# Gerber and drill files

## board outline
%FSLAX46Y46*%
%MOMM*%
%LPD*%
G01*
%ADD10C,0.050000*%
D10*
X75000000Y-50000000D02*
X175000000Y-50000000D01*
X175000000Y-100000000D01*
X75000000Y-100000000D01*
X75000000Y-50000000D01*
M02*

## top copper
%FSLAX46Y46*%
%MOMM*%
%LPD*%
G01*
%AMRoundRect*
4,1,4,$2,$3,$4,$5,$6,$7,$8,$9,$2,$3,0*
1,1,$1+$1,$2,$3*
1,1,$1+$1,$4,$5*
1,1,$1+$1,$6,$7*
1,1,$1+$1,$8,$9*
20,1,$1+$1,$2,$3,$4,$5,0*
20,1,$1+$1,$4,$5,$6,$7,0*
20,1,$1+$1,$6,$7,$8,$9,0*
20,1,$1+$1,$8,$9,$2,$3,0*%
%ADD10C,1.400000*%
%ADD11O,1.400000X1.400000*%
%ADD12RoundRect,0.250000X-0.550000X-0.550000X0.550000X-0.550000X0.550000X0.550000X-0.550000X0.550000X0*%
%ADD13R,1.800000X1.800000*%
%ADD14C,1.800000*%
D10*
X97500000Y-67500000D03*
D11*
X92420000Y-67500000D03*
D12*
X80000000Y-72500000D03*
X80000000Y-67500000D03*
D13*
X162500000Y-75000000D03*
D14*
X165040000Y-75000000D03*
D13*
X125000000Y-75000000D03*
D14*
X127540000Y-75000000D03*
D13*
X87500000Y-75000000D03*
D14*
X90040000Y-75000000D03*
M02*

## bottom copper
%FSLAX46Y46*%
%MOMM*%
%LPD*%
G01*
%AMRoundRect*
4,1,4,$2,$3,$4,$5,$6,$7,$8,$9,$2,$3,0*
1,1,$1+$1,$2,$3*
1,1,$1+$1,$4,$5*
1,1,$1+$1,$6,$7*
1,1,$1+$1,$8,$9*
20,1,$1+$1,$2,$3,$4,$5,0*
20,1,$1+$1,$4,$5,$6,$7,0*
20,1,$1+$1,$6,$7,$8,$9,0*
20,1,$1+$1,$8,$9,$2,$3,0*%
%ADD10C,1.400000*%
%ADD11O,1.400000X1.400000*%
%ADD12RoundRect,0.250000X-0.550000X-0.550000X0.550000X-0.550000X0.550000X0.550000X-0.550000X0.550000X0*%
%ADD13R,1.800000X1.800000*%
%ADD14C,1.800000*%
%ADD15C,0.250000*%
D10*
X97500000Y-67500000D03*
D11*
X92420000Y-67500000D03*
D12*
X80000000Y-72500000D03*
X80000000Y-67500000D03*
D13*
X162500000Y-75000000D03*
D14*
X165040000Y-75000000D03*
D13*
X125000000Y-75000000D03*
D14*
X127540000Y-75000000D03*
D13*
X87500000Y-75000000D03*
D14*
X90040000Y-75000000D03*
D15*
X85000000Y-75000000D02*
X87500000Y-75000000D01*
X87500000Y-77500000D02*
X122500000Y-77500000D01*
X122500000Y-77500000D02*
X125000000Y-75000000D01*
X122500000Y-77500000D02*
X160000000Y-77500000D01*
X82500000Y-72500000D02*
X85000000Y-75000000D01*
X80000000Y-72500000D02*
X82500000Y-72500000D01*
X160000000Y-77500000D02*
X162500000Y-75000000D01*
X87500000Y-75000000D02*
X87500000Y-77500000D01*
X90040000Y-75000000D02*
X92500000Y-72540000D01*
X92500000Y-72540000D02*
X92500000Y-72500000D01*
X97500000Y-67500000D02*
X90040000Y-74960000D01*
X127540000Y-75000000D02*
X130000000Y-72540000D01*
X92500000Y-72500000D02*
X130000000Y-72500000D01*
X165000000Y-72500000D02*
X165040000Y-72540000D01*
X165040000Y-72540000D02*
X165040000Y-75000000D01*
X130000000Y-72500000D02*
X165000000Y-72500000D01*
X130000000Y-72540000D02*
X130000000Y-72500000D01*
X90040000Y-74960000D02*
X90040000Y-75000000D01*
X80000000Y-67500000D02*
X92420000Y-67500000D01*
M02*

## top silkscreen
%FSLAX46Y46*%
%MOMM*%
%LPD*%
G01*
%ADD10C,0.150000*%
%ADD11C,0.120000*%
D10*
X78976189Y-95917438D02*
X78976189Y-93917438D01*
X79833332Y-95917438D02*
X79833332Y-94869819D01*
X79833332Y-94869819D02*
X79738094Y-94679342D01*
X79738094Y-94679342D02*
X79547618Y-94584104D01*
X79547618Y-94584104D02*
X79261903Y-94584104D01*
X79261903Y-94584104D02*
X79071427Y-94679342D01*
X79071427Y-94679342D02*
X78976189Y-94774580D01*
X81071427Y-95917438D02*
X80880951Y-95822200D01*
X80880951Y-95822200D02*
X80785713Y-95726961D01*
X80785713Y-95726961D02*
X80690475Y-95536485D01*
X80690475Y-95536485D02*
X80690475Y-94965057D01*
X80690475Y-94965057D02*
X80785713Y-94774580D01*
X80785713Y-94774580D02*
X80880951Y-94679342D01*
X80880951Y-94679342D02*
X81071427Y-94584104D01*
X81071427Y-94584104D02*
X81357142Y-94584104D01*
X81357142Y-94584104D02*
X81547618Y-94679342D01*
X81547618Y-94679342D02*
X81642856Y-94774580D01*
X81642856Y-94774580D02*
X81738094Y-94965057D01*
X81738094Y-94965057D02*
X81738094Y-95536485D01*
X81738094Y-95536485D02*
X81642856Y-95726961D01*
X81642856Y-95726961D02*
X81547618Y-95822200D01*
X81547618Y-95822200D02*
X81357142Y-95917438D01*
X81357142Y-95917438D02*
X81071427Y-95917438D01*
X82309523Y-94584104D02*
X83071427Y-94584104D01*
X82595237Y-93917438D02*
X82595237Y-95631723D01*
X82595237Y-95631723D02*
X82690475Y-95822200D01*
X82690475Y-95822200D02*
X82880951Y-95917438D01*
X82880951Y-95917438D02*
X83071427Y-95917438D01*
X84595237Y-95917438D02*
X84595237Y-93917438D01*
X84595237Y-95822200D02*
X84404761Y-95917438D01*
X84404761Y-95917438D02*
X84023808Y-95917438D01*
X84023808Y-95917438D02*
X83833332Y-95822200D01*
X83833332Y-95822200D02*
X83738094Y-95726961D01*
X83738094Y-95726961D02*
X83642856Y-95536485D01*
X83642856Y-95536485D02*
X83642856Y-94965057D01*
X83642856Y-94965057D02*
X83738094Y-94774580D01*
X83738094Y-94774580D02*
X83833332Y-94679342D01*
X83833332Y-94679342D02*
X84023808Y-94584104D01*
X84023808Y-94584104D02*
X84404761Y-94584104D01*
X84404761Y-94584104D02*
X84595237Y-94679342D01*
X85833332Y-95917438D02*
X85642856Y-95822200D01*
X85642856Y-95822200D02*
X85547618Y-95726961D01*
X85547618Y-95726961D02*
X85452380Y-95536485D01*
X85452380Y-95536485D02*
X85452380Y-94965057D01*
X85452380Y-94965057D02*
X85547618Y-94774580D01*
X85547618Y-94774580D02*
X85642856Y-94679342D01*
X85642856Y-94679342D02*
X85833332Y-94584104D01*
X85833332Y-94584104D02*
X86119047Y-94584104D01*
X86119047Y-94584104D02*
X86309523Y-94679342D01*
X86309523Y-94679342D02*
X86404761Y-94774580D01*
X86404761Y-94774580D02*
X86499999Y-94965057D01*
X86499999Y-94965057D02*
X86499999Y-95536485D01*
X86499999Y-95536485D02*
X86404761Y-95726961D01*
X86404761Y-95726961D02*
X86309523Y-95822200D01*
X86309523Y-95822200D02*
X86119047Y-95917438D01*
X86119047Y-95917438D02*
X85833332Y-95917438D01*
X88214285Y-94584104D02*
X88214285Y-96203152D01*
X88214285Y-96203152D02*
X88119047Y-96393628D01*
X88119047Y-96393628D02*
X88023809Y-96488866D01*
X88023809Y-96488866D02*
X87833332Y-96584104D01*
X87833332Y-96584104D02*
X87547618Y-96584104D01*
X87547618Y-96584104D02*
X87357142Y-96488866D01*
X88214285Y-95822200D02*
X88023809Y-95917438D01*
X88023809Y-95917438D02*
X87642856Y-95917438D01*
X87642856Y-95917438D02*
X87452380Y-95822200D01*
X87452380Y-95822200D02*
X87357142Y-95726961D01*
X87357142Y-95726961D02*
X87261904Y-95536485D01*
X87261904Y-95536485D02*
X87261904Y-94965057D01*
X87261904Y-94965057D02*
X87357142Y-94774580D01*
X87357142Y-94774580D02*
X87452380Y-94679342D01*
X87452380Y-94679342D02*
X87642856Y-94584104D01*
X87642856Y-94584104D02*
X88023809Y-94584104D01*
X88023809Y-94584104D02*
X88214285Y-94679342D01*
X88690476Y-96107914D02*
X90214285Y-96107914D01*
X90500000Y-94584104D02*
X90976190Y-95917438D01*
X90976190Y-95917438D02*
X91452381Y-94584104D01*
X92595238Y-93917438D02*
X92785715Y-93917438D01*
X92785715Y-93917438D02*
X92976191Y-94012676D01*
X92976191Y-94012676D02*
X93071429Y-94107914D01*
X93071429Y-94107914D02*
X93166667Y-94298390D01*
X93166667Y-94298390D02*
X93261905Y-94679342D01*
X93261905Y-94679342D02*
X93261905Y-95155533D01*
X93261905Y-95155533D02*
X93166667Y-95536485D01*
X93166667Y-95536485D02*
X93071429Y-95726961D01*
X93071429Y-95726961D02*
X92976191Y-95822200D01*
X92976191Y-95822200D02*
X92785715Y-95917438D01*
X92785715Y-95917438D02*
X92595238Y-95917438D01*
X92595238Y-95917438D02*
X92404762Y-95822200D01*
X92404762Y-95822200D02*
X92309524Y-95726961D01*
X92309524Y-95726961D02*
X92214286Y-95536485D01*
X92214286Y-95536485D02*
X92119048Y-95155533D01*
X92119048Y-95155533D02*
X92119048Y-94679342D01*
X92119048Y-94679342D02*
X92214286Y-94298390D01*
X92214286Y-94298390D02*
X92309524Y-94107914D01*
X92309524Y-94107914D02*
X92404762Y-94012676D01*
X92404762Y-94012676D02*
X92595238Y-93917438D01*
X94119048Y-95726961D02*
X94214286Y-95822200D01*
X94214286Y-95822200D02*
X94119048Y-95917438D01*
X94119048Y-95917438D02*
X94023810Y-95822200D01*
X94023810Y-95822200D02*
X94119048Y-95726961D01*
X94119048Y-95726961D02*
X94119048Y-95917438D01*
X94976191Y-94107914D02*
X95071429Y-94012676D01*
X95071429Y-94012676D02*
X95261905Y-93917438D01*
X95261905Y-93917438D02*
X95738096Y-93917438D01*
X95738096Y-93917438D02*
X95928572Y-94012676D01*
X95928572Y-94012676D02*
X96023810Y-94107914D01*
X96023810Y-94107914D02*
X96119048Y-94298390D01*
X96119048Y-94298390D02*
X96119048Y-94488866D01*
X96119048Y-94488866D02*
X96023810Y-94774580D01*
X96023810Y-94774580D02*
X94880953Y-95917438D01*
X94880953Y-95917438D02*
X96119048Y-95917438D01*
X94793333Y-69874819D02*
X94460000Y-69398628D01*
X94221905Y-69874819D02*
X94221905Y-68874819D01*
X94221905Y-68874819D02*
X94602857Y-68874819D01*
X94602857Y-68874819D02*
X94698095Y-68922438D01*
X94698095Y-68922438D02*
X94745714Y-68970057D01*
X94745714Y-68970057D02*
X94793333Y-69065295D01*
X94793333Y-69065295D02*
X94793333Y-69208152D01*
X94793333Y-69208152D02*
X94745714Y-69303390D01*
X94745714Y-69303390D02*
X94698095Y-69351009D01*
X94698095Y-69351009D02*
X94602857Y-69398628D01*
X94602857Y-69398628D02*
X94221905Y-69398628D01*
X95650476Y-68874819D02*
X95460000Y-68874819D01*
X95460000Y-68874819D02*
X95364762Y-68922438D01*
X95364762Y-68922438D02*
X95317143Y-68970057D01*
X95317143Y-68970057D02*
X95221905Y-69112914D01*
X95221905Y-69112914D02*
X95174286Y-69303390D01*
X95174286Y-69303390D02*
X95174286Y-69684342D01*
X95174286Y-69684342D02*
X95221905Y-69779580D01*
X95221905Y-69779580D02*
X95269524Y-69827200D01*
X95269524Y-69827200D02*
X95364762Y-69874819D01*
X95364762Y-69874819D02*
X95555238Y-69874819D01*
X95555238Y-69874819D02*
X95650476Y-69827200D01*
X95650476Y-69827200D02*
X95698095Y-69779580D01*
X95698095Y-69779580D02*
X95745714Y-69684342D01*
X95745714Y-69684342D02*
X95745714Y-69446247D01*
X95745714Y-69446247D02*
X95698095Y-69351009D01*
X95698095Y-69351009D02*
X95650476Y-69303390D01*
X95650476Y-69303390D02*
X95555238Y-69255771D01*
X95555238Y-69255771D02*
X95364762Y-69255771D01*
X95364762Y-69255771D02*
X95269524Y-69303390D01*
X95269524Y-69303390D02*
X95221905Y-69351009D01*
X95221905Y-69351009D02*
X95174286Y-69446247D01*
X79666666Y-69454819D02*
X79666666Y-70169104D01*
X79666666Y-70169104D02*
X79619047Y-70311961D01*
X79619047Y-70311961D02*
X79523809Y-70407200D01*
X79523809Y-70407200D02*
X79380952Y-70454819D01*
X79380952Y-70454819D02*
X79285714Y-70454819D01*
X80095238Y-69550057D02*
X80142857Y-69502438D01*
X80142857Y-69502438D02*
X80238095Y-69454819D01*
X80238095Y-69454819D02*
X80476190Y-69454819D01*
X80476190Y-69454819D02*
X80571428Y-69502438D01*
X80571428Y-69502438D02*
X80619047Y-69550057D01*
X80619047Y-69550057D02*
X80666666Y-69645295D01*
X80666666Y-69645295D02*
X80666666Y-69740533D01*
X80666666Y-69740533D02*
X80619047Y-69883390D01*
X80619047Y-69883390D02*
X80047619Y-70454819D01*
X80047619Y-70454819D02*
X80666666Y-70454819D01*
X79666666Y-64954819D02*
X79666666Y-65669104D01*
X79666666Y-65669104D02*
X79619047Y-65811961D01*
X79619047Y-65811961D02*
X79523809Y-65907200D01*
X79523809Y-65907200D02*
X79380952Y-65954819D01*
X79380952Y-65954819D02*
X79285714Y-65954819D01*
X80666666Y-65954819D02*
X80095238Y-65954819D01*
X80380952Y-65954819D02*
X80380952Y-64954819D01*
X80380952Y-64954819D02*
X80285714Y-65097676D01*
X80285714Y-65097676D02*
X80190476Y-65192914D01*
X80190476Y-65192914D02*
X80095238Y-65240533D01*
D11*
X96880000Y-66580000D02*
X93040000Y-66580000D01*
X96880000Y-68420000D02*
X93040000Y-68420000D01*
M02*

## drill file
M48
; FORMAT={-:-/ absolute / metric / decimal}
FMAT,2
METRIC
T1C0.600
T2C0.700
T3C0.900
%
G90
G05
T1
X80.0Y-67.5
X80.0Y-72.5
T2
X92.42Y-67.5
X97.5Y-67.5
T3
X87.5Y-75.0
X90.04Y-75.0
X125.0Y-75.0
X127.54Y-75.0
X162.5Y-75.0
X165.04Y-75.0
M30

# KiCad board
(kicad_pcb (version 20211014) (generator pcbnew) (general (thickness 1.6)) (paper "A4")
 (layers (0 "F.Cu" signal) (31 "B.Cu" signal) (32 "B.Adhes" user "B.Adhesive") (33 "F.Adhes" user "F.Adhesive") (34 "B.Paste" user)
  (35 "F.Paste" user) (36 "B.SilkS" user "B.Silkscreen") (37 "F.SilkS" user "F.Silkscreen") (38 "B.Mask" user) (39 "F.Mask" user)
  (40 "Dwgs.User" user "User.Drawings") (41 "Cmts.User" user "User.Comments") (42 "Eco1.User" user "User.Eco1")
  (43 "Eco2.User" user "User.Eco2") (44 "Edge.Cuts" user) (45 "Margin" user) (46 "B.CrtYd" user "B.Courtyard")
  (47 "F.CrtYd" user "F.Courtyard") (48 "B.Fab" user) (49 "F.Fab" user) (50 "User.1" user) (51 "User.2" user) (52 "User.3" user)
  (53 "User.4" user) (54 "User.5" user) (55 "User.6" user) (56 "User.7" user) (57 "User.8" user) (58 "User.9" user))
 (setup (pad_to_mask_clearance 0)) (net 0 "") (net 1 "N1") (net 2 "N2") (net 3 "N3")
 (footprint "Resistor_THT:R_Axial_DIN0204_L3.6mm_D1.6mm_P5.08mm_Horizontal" (layer "F.Cu") (at 97.5 67.5 180)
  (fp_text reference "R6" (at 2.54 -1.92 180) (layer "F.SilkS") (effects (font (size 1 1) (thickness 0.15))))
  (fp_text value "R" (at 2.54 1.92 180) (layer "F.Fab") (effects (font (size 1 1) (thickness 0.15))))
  (fp_line (start 0.62 0.92) (end 4.46 0.92) (layer "F.SilkS") (width 0.12))
  (fp_line (start 0.62 -0.92) (end 4.46 -0.92) (layer "F.SilkS") (width 0.12))
  (pad "1" thru_hole circle (at 0 0 180) (size 1.4 1.4) (drill 0.7) (layers *.Cu *.Mask) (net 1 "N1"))
  (pad "2" thru_hole oval (at 5.08 0 180) (size 1.4 1.4) (drill 0.7) (layers *.Cu *.Mask) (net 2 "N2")))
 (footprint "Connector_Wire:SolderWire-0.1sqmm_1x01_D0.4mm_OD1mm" (layer "F.Cu") (at 80 72.5)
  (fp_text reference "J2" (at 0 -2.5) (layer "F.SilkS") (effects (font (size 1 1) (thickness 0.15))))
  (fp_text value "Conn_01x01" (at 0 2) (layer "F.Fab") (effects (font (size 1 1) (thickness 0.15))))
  (pad "1" thru_hole roundrect (at 0 0) (size 1.6 1.6) (drill 0.6) (layers *.Cu *.Mask) (roundrect_rratio 0.15625) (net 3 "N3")))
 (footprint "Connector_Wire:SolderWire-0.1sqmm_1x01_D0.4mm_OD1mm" (layer "F.Cu") (at 80 67.5)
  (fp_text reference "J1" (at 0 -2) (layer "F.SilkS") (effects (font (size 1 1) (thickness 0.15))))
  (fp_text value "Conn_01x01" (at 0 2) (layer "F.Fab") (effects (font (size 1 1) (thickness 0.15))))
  (pad "1" thru_hole roundrect (at 0 0) (size 1.6 1.6) (drill 0.6) (layers *.Cu *.Mask) (roundrect_rratio 0.15625) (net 2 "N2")))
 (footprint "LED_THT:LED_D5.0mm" (layer "B.Cu") (at 162.5 75)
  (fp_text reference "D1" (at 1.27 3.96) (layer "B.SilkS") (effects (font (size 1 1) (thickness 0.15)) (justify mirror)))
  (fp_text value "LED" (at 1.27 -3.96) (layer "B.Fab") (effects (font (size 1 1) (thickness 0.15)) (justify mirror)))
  (pad "1" thru_hole rect (at 0 0) (size 1.8 1.8) (drill 0.9) (layers *.Cu *.Mask) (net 3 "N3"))
  (pad "2" thru_hole circle (at 2.54 0) (size 1.8 1.8) (drill 0.9) (layers *.Cu *.Mask) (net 1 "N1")))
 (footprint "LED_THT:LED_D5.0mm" (layer "B.Cu") (at 125 75)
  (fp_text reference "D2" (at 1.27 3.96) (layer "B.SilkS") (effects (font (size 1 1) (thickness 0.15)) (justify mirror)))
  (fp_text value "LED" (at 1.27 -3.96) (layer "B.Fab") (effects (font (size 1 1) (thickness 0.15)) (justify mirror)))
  (pad "1" thru_hole rect (at 0 0) (size 1.8 1.8) (drill 0.9) (layers *.Cu *.Mask) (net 3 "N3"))
  (pad "2" thru_hole circle (at 2.54 0) (size 1.8 1.8) (drill 0.9) (layers *.Cu *.Mask) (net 1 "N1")))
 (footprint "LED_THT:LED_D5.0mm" (layer "B.Cu") (at 87.5 75)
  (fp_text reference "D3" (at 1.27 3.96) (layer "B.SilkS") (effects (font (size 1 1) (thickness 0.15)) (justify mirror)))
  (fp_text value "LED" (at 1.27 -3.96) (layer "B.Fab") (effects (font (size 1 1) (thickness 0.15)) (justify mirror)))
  (pad "1" thru_hole rect (at 0 0) (size 1.8 1.8) (drill 0.9) (layers *.Cu *.Mask) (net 3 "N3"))
  (pad "2" thru_hole circle (at 2.54 0) (size 1.8 1.8) (drill 0.9) (layers *.Cu *.Mask) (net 1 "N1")))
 (gr_rect (start 175 50) (end 75 100) (layer "Edge.Cuts") (width 0.05) (fill none))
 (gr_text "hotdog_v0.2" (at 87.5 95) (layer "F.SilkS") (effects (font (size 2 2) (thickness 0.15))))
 (segment (start 85 75) (end 87.5 75) (width 0.25) (layer "B.Cu") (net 3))
 (segment (start 87.5 77.5) (end 122.5 77.5) (width 0.25) (layer "B.Cu") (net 3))
 (segment (start 122.5 77.5) (end 125 75) (width 0.25) (layer "B.Cu") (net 3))
 (segment (start 122.5 77.5) (end 160 77.5) (width 0.25) (layer "B.Cu") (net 3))
 (segment (start 82.5 72.5) (end 85 75) (width 0.25) (layer "B.Cu") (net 3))
 (segment (start 80 72.5) (end 82.5 72.5) (width 0.25) (layer "B.Cu") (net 3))
 (segment (start 160 77.5) (end 162.5 75) (width 0.25) (layer "B.Cu") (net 3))
 (segment (start 87.5 75) (end 87.5 77.5) (width 0.25) (layer "B.Cu") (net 3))
 (segment (start 90.04 75) (end 92.5 72.54) (width 0.25) (layer "B.Cu") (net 1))
 (segment (start 92.5 72.54) (end 92.5 72.5) (width 0.25) (layer "B.Cu") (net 1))
 (segment (start 97.5 67.5) (end 90.04 74.96) (width 0.25) (layer "B.Cu") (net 1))
 (segment (start 127.54 75) (end 130 72.54) (width 0.25) (layer "B.Cu") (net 1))
 (segment (start 92.5 72.5) (end 130 72.5) (width 0.25) (layer "B.Cu") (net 1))
 (segment (start 165 72.5) (end 165.04 72.54) (width 0.25) (layer "B.Cu") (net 1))
 (segment (start 165.04 72.54) (end 165.04 75) (width 0.25) (layer "B.Cu") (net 1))
 (segment (start 130 72.5) (end 165 72.5) (width 0.25) (layer "B.Cu") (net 1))
 (segment (start 130 72.54) (end 130 72.5) (width 0.25) (layer "B.Cu") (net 1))
 (segment (start 90.04 74.96) (end 90.04 75) (width 0.25) (layer "B.Cu") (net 1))
 (segment (start 80 67.5) (end 92.42 67.5) (width 0.25) (layer "B.Cu") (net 2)))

